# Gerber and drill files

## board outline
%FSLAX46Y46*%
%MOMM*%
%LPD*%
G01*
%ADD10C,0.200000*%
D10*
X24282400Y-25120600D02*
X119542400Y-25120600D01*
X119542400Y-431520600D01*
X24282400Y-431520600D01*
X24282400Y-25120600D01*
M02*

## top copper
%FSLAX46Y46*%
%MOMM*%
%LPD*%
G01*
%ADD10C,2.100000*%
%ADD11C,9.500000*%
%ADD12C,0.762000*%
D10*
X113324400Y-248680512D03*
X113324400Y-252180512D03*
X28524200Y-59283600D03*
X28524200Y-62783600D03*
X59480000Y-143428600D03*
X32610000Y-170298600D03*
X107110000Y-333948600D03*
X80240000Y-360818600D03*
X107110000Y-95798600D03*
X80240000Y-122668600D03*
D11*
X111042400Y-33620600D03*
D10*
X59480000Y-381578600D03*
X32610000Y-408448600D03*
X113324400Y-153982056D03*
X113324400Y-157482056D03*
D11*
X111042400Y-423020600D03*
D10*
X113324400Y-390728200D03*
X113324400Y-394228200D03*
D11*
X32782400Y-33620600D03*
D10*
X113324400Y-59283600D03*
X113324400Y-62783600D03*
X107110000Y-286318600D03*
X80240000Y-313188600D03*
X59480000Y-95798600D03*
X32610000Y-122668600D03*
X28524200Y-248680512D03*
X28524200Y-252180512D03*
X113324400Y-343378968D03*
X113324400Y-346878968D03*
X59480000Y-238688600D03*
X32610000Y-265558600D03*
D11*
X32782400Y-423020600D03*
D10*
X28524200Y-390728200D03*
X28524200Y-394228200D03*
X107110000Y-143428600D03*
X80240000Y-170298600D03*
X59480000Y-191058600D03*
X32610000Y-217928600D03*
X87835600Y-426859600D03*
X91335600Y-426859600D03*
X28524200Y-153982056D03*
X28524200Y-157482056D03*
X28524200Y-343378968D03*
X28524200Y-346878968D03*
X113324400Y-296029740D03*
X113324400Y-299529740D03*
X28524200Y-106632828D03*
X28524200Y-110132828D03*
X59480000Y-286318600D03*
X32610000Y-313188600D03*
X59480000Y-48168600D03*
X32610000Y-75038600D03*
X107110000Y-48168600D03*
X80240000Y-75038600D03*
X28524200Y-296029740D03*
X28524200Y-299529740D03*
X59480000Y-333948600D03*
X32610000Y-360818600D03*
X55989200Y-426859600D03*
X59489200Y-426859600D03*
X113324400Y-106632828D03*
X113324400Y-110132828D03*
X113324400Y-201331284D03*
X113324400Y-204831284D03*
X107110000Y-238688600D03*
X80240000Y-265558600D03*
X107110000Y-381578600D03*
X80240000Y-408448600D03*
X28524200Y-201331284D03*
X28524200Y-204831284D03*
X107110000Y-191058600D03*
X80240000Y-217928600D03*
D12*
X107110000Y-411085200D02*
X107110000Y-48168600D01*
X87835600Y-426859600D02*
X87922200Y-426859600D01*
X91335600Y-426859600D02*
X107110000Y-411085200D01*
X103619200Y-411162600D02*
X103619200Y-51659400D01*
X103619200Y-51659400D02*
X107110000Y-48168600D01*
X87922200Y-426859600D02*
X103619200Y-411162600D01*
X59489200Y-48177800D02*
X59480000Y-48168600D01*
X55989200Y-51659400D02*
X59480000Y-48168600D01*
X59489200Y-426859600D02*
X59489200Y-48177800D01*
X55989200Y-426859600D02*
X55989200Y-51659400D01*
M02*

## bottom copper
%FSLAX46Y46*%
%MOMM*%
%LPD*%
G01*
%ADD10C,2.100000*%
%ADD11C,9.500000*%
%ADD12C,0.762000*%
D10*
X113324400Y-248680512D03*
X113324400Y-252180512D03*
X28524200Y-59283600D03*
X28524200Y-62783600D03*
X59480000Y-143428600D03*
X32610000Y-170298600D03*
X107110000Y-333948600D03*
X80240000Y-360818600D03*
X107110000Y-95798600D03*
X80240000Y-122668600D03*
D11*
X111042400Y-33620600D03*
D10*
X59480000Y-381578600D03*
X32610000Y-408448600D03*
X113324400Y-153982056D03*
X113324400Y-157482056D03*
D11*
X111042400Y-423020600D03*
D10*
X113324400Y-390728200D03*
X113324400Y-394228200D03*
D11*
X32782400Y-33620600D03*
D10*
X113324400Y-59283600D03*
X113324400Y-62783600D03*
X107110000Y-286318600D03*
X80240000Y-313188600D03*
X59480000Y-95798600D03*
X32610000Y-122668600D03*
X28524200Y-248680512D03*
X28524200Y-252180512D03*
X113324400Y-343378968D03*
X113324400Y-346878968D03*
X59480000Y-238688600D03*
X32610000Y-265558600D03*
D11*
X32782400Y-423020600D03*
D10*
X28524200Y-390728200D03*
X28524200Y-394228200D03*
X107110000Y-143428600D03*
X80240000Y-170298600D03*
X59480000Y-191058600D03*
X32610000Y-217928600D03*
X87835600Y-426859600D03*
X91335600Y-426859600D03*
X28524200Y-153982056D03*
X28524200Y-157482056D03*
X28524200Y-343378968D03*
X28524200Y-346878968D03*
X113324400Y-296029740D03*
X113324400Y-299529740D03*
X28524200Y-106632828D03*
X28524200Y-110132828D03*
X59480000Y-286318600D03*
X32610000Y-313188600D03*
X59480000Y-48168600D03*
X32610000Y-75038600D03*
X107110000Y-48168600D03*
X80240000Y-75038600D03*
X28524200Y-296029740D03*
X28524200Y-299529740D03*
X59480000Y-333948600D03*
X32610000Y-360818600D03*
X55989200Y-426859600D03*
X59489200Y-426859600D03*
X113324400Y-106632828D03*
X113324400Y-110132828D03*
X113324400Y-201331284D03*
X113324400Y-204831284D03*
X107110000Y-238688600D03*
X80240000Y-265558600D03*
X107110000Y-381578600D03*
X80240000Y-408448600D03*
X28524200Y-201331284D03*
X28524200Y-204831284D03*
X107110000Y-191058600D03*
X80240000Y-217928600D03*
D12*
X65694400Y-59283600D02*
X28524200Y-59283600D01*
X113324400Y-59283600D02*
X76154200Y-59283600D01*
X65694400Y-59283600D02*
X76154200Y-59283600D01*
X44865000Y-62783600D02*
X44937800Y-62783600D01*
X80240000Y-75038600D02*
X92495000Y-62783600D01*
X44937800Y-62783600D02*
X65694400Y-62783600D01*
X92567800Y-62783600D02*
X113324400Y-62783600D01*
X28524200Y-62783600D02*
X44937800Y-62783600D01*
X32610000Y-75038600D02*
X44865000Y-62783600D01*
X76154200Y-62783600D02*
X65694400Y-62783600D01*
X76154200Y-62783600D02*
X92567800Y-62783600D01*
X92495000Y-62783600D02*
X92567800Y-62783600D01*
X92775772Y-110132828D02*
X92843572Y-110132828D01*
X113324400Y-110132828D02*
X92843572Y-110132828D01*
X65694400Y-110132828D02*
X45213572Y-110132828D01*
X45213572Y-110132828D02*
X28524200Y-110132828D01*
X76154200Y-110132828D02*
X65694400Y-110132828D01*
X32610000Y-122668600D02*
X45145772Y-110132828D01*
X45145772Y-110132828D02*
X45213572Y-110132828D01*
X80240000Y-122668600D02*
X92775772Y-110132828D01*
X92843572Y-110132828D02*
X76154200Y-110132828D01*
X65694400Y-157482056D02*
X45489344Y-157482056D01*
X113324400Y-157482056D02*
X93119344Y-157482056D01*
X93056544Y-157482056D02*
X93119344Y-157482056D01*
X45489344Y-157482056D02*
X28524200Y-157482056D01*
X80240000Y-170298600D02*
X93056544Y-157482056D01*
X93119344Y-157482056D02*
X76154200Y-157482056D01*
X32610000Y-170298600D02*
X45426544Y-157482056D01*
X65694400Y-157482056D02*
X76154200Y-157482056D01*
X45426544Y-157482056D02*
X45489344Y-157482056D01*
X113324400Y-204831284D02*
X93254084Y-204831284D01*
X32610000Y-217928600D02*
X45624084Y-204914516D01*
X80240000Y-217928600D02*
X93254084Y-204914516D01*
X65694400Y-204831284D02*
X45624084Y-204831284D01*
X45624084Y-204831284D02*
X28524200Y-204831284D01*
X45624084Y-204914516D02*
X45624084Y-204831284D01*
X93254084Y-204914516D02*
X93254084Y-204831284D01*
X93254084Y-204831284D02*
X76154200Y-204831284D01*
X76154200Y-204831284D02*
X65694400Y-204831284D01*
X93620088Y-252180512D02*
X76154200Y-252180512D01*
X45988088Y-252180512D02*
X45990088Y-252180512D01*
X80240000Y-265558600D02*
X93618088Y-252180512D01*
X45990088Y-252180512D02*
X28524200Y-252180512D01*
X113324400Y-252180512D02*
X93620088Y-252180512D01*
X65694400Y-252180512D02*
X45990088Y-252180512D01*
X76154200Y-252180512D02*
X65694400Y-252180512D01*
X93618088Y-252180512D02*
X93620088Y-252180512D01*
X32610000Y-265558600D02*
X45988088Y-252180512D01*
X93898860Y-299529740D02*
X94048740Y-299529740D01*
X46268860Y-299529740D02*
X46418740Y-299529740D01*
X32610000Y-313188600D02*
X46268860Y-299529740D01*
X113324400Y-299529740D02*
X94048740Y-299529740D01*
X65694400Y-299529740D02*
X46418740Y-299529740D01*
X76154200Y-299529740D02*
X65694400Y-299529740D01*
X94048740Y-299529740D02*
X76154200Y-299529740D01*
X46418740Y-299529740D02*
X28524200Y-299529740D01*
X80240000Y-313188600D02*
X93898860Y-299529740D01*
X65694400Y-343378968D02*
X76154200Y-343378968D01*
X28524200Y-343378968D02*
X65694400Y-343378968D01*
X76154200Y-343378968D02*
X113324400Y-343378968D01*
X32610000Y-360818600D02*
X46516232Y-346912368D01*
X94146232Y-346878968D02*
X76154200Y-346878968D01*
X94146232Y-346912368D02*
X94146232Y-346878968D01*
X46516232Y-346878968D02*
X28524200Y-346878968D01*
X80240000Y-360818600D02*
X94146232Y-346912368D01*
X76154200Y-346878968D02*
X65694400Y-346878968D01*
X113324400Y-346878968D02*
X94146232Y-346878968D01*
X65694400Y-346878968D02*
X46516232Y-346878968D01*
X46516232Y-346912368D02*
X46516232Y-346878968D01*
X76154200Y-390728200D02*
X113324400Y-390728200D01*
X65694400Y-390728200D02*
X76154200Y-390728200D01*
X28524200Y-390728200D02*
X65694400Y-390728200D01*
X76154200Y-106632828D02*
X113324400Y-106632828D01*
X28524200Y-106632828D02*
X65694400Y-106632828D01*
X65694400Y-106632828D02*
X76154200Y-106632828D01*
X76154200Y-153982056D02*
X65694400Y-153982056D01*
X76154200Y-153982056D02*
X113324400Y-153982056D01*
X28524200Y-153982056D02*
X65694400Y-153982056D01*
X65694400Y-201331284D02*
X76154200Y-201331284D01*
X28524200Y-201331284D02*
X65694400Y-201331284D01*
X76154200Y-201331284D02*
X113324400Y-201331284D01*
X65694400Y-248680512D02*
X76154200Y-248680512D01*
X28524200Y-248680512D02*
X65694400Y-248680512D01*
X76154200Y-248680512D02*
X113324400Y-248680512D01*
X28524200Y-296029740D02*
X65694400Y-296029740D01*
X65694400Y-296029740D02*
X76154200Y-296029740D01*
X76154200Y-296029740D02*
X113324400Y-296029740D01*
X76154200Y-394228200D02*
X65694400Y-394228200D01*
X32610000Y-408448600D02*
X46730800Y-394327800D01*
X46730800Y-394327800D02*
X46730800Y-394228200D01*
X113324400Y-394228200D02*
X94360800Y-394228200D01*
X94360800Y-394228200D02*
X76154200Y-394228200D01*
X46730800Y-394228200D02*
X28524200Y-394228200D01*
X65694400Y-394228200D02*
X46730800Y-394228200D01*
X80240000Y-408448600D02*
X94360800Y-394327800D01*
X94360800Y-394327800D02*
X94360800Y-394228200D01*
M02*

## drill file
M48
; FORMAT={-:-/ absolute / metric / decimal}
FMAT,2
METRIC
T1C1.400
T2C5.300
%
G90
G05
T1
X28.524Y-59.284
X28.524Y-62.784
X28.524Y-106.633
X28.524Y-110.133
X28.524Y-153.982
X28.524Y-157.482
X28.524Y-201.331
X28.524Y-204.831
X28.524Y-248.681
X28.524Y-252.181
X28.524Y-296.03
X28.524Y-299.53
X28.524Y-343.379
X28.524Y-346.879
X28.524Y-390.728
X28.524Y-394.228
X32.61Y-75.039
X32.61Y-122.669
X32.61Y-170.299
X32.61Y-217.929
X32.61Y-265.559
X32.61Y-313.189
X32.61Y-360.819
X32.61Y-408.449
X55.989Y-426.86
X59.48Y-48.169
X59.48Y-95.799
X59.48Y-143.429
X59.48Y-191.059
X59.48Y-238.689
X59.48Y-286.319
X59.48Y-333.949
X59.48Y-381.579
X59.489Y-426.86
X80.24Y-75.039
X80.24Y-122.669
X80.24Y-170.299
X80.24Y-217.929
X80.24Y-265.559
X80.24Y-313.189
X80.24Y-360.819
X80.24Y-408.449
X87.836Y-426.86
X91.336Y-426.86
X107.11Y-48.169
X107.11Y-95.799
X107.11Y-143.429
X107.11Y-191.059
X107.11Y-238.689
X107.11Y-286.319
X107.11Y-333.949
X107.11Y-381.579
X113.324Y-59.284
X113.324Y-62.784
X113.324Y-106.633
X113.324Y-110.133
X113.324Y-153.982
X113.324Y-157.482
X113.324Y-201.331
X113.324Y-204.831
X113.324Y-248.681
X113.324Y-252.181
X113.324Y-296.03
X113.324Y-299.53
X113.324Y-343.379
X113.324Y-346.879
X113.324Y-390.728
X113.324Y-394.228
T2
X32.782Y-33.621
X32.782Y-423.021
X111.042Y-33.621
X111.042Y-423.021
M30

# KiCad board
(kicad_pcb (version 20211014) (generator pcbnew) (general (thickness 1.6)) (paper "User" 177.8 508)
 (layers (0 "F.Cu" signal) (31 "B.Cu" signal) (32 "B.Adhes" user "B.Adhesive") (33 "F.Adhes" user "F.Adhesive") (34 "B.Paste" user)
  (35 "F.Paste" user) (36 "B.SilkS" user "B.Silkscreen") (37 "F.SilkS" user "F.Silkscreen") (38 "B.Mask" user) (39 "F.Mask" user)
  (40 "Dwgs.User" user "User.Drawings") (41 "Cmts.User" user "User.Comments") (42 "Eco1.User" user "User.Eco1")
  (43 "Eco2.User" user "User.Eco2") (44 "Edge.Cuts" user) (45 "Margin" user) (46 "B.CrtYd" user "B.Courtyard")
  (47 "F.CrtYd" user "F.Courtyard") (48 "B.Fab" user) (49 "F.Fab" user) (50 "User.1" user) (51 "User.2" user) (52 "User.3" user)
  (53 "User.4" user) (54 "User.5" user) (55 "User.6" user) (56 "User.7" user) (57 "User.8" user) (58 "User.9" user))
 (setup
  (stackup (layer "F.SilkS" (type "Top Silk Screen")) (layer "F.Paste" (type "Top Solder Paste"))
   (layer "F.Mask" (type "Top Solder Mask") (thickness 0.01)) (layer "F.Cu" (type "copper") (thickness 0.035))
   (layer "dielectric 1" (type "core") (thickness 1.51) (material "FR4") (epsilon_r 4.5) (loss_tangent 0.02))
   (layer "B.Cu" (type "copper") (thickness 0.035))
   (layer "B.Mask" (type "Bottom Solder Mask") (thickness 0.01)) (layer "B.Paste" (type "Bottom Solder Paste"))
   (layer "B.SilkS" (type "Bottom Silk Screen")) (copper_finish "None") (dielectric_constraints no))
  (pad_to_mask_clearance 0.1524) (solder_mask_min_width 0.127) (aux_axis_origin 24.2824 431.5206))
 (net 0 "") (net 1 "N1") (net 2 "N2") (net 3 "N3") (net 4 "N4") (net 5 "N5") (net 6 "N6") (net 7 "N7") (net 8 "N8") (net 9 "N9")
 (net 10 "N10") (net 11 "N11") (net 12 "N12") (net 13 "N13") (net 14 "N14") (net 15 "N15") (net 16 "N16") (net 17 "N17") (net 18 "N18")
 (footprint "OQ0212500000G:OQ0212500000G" (layer "F.Cu") (at 113.3244 248.680512 -90)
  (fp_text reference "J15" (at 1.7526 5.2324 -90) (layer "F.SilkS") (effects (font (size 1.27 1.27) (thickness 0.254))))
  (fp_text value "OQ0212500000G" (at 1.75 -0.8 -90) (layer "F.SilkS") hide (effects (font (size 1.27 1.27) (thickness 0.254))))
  (pad "1" thru_hole circle (at 0 0 270) (size 2.1 2.1) (drill 1.4) (layers F&B.Cu *.Mask) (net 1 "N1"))
  (pad "2" thru_hole circle (at 3.5 0 270) (size 2.1 2.1) (drill 1.4) (layers F&B.Cu *.Mask) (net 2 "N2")))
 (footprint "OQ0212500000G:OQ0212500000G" (layer "F.Cu") (at 28.5242 59.2836 -90)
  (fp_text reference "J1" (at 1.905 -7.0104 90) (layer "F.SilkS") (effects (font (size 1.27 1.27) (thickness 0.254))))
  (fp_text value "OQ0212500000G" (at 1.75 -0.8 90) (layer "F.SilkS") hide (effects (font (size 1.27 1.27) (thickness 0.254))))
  (pad "1" thru_hole circle (at 0 0 270) (size 2.1 2.1) (drill 1.4) (layers *.Cu *.Mask) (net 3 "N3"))
  (pad "2" thru_hole circle (at 3.5 0 270) (size 2.1 2.1) (drill 1.4) (layers *.Cu *.Mask) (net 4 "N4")))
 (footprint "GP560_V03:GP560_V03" (layer "F.Cu") (at 32.61 170.2986)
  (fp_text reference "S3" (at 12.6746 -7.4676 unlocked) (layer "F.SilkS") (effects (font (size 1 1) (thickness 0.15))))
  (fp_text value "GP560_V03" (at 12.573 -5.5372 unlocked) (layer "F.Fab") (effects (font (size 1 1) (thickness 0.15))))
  (pad "1" thru_hole circle (at 26.87 -26.87) (size 2.1 2.1) (drill 1.4) (layers *.Cu *.Mask) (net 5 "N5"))
  (pad "2" thru_hole circle (at 0 0) (size 2.1 2.1) (drill 1.4) (layers *.Cu *.Mask) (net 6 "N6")))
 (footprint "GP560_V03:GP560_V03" (layer "F.Cu") (at 80.24 360.8186)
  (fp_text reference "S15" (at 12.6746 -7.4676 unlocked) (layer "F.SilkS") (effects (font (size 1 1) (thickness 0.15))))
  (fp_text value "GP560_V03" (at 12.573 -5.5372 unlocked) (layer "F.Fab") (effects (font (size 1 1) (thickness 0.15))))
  (pad "1" thru_hole circle (at 26.87 -26.87) (size 2.1 2.1) (drill 1.4) (layers *.Cu *.Mask) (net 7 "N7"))
  (pad "2" thru_hole circle (at 0 0) (size 2.1 2.1) (drill 1.4) (layers *.Cu *.Mask) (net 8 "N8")))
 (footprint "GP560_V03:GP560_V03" (layer "F.Cu") (at 80.24 122.6686)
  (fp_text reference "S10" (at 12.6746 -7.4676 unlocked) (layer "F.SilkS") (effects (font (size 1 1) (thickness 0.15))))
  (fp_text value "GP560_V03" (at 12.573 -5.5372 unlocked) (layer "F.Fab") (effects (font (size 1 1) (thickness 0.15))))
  (pad "1" thru_hole circle (at 26.87 -26.87) (size 2.1 2.1) (drill 1.4) (layers *.Cu *.Mask) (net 7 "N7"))
  (pad "2" thru_hole circle (at 0 0) (size 2.1 2.1) (drill 1.4) (layers *.Cu *.Mask) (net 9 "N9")))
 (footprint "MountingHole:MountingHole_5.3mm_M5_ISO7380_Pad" (layer "F.Cu") (at 111.0424 33.6206)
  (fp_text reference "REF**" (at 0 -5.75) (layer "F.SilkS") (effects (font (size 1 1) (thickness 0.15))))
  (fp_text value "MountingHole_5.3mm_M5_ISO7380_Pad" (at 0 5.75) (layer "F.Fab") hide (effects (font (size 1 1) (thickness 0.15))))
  (pad "1" thru_hole circle (at 0 0) (size 9.5 9.5) (drill 5.3) (layers F&B.Cu *.Mask)))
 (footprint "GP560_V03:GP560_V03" (layer "F.Cu") (at 32.61 408.4486)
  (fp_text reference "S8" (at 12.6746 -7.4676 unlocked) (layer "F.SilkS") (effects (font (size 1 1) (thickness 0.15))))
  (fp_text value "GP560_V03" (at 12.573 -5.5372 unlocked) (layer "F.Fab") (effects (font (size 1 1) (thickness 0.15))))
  (pad "1" thru_hole circle (at 26.87 -26.87) (size 2.1 2.1) (drill 1.4) (layers *.Cu *.Mask) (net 5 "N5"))
  (pad "2" thru_hole circle (at 0 0) (size 2.1 2.1) (drill 1.4) (layers *.Cu *.Mask) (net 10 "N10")))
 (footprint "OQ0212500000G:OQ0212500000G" (layer "F.Cu") (at 113.3244 153.982056 -90)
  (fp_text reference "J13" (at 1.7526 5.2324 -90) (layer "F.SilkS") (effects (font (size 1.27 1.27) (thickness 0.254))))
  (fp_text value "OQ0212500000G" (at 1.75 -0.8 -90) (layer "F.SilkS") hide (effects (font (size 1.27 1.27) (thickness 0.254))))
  (pad "1" thru_hole circle (at 0 0 270) (size 2.1 2.1) (drill 1.4) (layers F&B.Cu *.Mask) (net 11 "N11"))
  (pad "2" thru_hole circle (at 3.5 0 270) (size 2.1 2.1) (drill 1.4) (layers F&B.Cu *.Mask) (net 6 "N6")))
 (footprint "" (layer "F.Cu") (at 111.0424 423.0206)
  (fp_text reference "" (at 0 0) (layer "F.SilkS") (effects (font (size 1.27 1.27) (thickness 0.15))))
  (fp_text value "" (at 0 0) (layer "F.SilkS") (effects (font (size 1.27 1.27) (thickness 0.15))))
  (pad "1" thru_hole circle (at 0 0) (size 9.5 9.5) (drill 5.3) (layers F&B.Cu *.Mask)))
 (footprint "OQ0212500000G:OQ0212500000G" (layer "F.Cu") (at 113.3244 390.7282 -90)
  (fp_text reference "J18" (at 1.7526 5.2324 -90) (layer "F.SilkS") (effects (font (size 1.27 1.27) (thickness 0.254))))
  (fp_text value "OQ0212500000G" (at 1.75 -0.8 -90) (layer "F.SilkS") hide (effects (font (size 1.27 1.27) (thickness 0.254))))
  (pad "1" thru_hole circle (at 0 0 270) (size 2.1 2.1) (drill 1.4) (layers F&B.Cu *.Mask) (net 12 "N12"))
  (pad "2" thru_hole circle (at 3.5 0 270) (size 2.1 2.1) (drill 1.4) (layers F&B.Cu *.Mask) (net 10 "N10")))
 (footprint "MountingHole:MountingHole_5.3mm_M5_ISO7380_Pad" (layer "F.Cu") (at 32.7824 33.6206)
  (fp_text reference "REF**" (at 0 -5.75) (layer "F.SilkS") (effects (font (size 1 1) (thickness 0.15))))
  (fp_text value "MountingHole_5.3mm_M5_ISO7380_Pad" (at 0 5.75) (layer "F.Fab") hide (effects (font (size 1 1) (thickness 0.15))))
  (pad "1" thru_hole circle (at 0 0) (size 9.5 9.5) (drill 5.3) (layers F&B.Cu *.Mask)))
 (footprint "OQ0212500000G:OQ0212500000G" (layer "F.Cu") (at 113.3244 59.2836 -90)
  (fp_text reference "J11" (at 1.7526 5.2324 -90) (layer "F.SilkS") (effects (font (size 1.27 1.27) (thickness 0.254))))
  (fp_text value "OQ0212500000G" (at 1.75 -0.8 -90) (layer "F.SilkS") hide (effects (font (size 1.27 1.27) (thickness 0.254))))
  (pad "1" thru_hole circle (at 0 0 270) (size 2.1 2.1) (drill 1.4) (layers F&B.Cu *.Mask) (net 3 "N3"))
  (pad "2" thru_hole circle (at 3.5 0 270) (size 2.1 2.1) (drill 1.4) (layers F&B.Cu *.Mask) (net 4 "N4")))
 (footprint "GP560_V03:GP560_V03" (layer "F.Cu") (at 80.24 313.1886)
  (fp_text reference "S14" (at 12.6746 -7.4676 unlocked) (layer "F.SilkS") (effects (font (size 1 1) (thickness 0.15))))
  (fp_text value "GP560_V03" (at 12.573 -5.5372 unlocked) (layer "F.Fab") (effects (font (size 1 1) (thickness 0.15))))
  (pad "1" thru_hole circle (at 26.87 -26.87) (size 2.1 2.1) (drill 1.4) (layers *.Cu *.Mask) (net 7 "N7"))
  (pad "2" thru_hole circle (at 0 0) (size 2.1 2.1) (drill 1.4) (layers *.Cu *.Mask) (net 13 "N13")))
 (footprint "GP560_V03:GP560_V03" (layer "F.Cu") (at 32.61 122.6686)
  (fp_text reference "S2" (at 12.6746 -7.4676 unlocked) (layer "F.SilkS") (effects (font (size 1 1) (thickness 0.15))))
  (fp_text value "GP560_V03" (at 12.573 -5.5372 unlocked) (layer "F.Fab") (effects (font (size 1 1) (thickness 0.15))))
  (pad "1" thru_hole circle (at 26.87 -26.87) (size 2.1 2.1) (drill 1.4) (layers *.Cu *.Mask) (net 5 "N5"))
  (pad "2" thru_hole circle (at 0 0) (size 2.1 2.1) (drill 1.4) (layers *.Cu *.Mask) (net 9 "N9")))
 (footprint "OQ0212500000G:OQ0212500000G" (layer "F.Cu") (at 28.5242 248.680512 -90)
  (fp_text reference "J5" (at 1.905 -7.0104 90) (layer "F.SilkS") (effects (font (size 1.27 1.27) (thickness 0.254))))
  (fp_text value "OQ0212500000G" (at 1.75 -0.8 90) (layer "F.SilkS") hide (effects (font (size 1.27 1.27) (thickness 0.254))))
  (pad "1" thru_hole circle (at 0 0 270) (size 2.1 2.1) (drill 1.4) (layers *.Cu *.Mask) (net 1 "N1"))
  (pad "2" thru_hole circle (at 3.5 0 270) (size 2.1 2.1) (drill 1.4) (layers *.Cu *.Mask) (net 2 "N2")))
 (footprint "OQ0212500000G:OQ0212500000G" (layer "F.Cu") (at 113.3244 343.378968 -90)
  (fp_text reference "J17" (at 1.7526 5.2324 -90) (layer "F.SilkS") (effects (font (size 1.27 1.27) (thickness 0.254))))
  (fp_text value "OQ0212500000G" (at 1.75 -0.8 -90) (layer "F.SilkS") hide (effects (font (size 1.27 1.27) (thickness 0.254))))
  (pad "1" thru_hole circle (at 0 0 270) (size 2.1 2.1) (drill 1.4) (layers F&B.Cu *.Mask) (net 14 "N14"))
  (pad "2" thru_hole circle (at 3.5 0 270) (size 2.1 2.1) (drill 1.4) (layers F&B.Cu *.Mask) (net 8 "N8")))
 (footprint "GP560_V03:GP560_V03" (layer "F.Cu") (at 32.61 265.5586)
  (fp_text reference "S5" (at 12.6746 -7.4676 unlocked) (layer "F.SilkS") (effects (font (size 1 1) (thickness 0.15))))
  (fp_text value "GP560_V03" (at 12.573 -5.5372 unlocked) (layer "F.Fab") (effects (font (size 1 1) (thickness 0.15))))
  (pad "1" thru_hole circle (at 26.87 -26.87) (size 2.1 2.1) (drill 1.4) (layers *.Cu *.Mask) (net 5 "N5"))
  (pad "2" thru_hole circle (at 0 0) (size 2.1 2.1) (drill 1.4) (layers *.Cu *.Mask) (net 2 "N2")))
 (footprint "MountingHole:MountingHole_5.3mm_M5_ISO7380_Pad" (layer "F.Cu") (at 32.7824 423.0206)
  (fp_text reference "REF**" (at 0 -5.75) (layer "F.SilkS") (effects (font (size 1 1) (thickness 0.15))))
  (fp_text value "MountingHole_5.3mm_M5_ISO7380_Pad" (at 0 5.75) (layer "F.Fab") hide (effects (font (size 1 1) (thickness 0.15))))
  (pad "1" thru_hole circle (at 0 0) (size 9.5 9.5) (drill 5.3) (layers *.Cu *.Mask)))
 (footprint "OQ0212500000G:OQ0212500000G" (layer "F.Cu") (at 28.5242 390.7282 -90)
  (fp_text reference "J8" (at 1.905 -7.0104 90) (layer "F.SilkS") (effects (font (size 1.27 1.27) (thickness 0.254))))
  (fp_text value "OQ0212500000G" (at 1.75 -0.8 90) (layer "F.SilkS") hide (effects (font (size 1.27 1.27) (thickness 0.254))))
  (pad "1" thru_hole circle (at 0 0 270) (size 2.1 2.1) (drill 1.4) (layers *.Cu *.Mask) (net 12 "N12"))
  (pad "2" thru_hole circle (at 3.5 0 270) (size 2.1 2.1) (drill 1.4) (layers *.Cu *.Mask) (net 10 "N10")))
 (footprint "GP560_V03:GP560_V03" (layer "F.Cu") (at 80.24 170.2986)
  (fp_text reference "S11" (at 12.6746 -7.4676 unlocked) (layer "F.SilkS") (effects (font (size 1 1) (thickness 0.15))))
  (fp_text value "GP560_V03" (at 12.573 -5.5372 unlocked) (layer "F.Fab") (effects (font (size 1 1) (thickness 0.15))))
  (pad "1" thru_hole circle (at 26.87 -26.87) (size 2.1 2.1) (drill 1.4) (layers *.Cu *.Mask) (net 7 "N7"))
  (pad "2" thru_hole circle (at 0 0) (size 2.1 2.1) (drill 1.4) (layers *.Cu *.Mask) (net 6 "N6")))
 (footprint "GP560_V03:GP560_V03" (layer "F.Cu") (at 32.61 217.9286)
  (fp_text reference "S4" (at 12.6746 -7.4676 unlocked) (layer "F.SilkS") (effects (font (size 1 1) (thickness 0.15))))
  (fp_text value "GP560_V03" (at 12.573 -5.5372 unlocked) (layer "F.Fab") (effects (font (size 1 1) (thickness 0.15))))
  (pad "1" thru_hole circle (at 26.87 -26.87) (size 2.1 2.1) (drill 1.4) (layers *.Cu *.Mask) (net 5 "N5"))
  (pad "2" thru_hole circle (at 0 0) (size 2.1 2.1) (drill 1.4) (layers *.Cu *.Mask) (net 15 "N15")))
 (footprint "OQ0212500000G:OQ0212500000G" (layer "F.Cu") (at 87.8356 426.8596)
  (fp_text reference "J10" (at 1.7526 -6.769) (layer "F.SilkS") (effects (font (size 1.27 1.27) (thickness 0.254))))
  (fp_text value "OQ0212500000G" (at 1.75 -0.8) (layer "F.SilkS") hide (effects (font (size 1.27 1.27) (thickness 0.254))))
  (pad "1" thru_hole circle (at 0 0) (size 2.1 2.1) (drill 1.4) (layers *.Cu *.Mask) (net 7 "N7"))
  (pad "2" thru_hole circle (at 3.5 0) (size 2.1 2.1) (drill 1.4) (layers *.Cu *.Mask) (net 7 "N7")))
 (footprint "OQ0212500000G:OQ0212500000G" (layer "F.Cu") (at 28.5242 153.982056 -90)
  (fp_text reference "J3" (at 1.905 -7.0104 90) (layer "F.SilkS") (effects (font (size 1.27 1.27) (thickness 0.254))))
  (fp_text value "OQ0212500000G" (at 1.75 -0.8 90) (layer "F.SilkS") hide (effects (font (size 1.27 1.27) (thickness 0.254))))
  (pad "1" thru_hole circle (at 0 0 270) (size 2.1 2.1) (drill 1.4) (layers *.Cu *.Mask) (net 11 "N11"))
  (pad "2" thru_hole circle (at 3.5 0 270) (size 2.1 2.1) (drill 1.4) (layers *.Cu *.Mask) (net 6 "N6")))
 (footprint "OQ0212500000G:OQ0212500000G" (layer "F.Cu") (at 28.5242 343.378968 -90)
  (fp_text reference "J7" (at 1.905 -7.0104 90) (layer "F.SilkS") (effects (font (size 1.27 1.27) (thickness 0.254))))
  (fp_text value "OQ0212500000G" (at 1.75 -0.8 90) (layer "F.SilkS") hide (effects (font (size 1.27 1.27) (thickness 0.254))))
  (pad "1" thru_hole circle (at 0 0 270) (size 2.1 2.1) (drill 1.4) (layers *.Cu *.Mask) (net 14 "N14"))
  (pad "2" thru_hole circle (at 3.5 0 270) (size 2.1 2.1) (drill 1.4) (layers *.Cu *.Mask) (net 8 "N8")))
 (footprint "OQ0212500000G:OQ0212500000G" (layer "F.Cu") (at 113.3244 296.02974 -90)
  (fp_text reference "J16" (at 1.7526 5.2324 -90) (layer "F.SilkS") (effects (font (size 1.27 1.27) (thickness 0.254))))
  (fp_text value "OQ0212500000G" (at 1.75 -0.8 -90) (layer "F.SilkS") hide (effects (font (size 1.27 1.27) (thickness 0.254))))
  (pad "1" thru_hole circle (at 0 0 270) (size 2.1 2.1) (drill 1.4) (layers F&B.Cu *.Mask) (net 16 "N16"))
  (pad "2" thru_hole circle (at 3.5 0 270) (size 2.1 2.1) (drill 1.4) (layers F&B.Cu *.Mask) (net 13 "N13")))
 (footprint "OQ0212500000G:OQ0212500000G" (layer "F.Cu") (at 28.5242 106.632828 -90)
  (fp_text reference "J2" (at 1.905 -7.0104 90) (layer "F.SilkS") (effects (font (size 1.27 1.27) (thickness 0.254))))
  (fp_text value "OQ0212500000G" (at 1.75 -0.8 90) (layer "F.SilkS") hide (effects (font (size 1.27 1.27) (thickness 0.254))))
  (pad "1" thru_hole circle (at 0 0 270) (size 2.1 2.1) (drill 1.4) (layers *.Cu *.Mask) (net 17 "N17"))
  (pad "2" thru_hole circle (at 3.5 0 270) (size 2.1 2.1) (drill 1.4) (layers *.Cu *.Mask) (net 9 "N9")))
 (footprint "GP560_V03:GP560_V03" (layer "F.Cu") (at 32.61 313.1886)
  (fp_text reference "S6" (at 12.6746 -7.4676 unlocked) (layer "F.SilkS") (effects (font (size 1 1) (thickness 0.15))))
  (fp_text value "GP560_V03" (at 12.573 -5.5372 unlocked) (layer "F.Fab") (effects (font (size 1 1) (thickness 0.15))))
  (pad "1" thru_hole circle (at 26.87 -26.87) (size 2.1 2.1) (drill 1.4) (layers *.Cu *.Mask) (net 5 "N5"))
  (pad "2" thru_hole circle (at 0 0) (size 2.1 2.1) (drill 1.4) (layers *.Cu *.Mask) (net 13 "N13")))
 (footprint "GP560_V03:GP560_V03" (layer "F.Cu") (at 32.61 75.0386)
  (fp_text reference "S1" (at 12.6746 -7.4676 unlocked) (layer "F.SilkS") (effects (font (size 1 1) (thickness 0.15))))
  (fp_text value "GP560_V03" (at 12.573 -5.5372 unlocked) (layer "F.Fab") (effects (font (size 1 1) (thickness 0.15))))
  (pad "1" thru_hole circle (at 26.87 -26.87) (size 2.1 2.1) (drill 1.4) (layers *.Cu *.Mask) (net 5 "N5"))
  (pad "2" thru_hole circle (at 0 0) (size 2.1 2.1) (drill 1.4) (layers *.Cu *.Mask) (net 4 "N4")))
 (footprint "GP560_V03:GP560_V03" (layer "F.Cu") (at 80.24 75.0386)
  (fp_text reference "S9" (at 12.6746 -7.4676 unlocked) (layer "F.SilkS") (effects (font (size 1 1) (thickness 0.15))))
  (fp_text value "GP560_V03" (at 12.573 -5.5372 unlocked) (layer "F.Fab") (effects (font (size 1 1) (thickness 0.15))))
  (pad "1" thru_hole circle (at 26.87 -26.87) (size 2.1 2.1) (drill 1.4) (layers *.Cu *.Mask) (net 7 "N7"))
  (pad "2" thru_hole circle (at 0 0) (size 2.1 2.1) (drill 1.4) (layers *.Cu *.Mask) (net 4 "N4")))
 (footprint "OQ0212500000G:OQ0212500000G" (layer "F.Cu") (at 28.5242 296.02974 -90)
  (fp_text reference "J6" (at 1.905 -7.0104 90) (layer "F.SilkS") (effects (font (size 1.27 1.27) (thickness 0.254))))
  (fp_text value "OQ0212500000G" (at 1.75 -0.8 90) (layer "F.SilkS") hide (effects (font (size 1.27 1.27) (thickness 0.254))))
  (pad "1" thru_hole circle (at 0 0 270) (size 2.1 2.1) (drill 1.4) (layers *.Cu *.Mask) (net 16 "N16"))
  (pad "2" thru_hole circle (at 3.5 0 270) (size 2.1 2.1) (drill 1.4) (layers *.Cu *.Mask) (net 13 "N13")))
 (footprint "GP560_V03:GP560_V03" (layer "F.Cu") (at 32.61 360.8186)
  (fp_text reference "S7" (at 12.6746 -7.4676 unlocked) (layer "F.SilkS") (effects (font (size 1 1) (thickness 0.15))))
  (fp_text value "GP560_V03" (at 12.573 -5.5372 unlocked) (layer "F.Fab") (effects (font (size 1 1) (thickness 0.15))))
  (pad "1" thru_hole circle (at 26.87 -26.87) (size 2.1 2.1) (drill 1.4) (layers *.Cu *.Mask) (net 5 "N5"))
  (pad "2" thru_hole circle (at 0 0) (size 2.1 2.1) (drill 1.4) (layers *.Cu *.Mask) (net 8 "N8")))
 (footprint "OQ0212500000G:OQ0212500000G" (layer "F.Cu") (at 55.9892 426.8596)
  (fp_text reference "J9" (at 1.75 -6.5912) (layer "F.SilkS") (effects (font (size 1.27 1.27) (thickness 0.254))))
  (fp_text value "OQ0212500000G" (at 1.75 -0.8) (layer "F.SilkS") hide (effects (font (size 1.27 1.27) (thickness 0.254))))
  (pad "1" thru_hole circle (at 0 0) (size 2.1 2.1) (drill 1.4) (layers *.Cu *.Mask) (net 5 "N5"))
  (pad "2" thru_hole circle (at 3.5 0) (size 2.1 2.1) (drill 1.4) (layers *.Cu *.Mask) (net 5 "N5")))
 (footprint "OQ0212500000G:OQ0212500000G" (layer "F.Cu") (at 113.3244 106.632828 -90)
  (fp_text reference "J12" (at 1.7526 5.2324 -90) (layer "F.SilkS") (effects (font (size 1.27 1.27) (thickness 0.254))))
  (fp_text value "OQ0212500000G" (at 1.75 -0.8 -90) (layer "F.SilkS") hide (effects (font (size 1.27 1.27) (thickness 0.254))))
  (pad "1" thru_hole circle (at 0 0 270) (size 2.1 2.1) (drill 1.4) (layers F&B.Cu *.Mask) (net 17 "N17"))
  (pad "2" thru_hole circle (at 3.5 0 270) (size 2.1 2.1) (drill 1.4) (layers F&B.Cu *.Mask) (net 9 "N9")))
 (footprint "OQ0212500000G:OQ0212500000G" (layer "F.Cu") (at 113.3244 201.331284 -90)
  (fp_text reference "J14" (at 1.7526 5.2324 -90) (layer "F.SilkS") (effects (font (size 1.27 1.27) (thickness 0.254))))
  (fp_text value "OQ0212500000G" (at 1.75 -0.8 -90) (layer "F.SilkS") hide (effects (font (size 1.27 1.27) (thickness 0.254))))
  (pad "1" thru_hole circle (at 0 0 270) (size 2.1 2.1) (drill 1.4) (layers F&B.Cu *.Mask) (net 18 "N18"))
  (pad "2" thru_hole circle (at 3.5 0 270) (size 2.1 2.1) (drill 1.4) (layers F&B.Cu *.Mask) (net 15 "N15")))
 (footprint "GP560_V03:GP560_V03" (layer "F.Cu") (at 80.24 265.5586)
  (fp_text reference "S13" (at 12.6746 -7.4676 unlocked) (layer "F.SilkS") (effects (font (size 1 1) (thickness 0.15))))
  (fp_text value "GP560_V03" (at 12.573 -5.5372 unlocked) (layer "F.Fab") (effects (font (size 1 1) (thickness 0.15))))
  (pad "1" thru_hole circle (at 26.87 -26.87) (size 2.1 2.1) (drill 1.4) (layers *.Cu *.Mask) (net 7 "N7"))
  (pad "2" thru_hole circle (at 0 0) (size 2.1 2.1) (drill 1.4) (layers *.Cu *.Mask) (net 2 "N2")))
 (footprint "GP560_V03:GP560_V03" (layer "F.Cu") (at 80.24 408.4486)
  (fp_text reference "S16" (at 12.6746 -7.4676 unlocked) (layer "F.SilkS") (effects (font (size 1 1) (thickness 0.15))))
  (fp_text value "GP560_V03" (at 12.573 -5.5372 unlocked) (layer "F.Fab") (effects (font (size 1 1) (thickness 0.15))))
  (pad "1" thru_hole circle (at 26.87 -26.87) (size 2.1 2.1) (drill 1.4) (layers *.Cu *.Mask) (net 7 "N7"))
  (pad "2" thru_hole circle (at 0 0) (size 2.1 2.1) (drill 1.4) (layers *.Cu *.Mask) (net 10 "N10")))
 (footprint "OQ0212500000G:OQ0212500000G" (layer "F.Cu") (at 28.5242 201.331284 -90)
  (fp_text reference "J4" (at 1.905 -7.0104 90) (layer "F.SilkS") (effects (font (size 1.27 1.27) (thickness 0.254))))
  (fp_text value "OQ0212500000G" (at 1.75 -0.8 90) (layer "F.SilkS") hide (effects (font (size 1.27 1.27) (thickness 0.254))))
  (pad "1" thru_hole circle (at 0 0 270) (size 2.1 2.1) (drill 1.4) (layers *.Cu *.Mask) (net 18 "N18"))
  (pad "2" thru_hole circle (at 3.5 0 270) (size 2.1 2.1) (drill 1.4) (layers *.Cu *.Mask) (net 15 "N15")))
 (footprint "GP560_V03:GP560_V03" (layer "F.Cu") (at 80.24 217.9286)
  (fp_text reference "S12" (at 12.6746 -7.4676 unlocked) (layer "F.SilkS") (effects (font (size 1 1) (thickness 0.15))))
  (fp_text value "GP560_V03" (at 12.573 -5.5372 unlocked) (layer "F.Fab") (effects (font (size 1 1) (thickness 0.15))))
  (pad "1" thru_hole circle (at 26.87 -26.87) (size 2.1 2.1) (drill 1.4) (layers *.Cu *.Mask) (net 7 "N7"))
  (pad "2" thru_hole circle (at 0 0) (size 2.1 2.1) (drill 1.4) (layers *.Cu *.Mask) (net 15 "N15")))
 (gr_rect (start 24.2824 431.5206) (end 119.5424 25.1206) (layer "Edge.Cuts") (width 0.2) (fill none))
 (segment (start 65.6944 59.2836) (end 28.5242 59.2836) (width 0.762) (layer "B.Cu") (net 3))
 (segment (start 113.3244 59.2836) (end 76.1542 59.2836) (width 0.762) (layer "B.Cu") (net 3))
 (segment (start 65.6944 59.2836) (end 76.1542 59.2836) (width 0.762) (layer "B.Cu") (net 3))
 (segment (start 44.865 62.7836) (end 44.9378 62.7836) (width 0.762) (layer "B.Cu") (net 4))
 (segment (start 80.24 75.0386) (end 92.495 62.7836) (width 0.762) (layer "B.Cu") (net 4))
 (segment (start 44.9378 62.7836) (end 65.6944 62.7836) (width 0.762) (layer "B.Cu") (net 4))
 (segment (start 92.5678 62.7836) (end 113.3244 62.7836) (width 0.762) (layer "B.Cu") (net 4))
 (segment (start 28.5242 62.7836) (end 44.9378 62.7836) (width 0.762) (layer "B.Cu") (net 4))
 (segment (start 32.61 75.0386) (end 44.865 62.7836) (width 0.762) (layer "B.Cu") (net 4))
 (segment (start 76.1542 62.7836) (end 65.6944 62.7836) (width 0.762) (layer "B.Cu") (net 4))
 (segment (start 76.1542 62.7836) (end 92.5678 62.7836) (width 0.762) (layer "B.Cu") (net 4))
 (segment (start 92.495 62.7836) (end 92.5678 62.7836) (width 0.762) (layer "B.Cu") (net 4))
 (segment (start 92.775772 110.132828) (end 92.843572 110.132828) (width 0.762) (layer "B.Cu") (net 9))
 (segment (start 113.3244 110.132828) (end 92.843572 110.132828) (width 0.762) (layer "B.Cu") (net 9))
 (segment (start 65.6944 110.132828) (end 45.213572 110.132828) (width 0.762) (layer "B.Cu") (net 9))
 (segment (start 45.213572 110.132828) (end 28.5242 110.132828) (width 0.762) (layer "B.Cu") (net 9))
 (segment (start 76.1542 110.132828) (end 65.6944 110.132828) (width 0.762) (layer "B.Cu") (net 9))
 (segment (start 32.61 122.6686) (end 45.145772 110.132828) (width 0.762) (layer "B.Cu") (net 9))
 (segment (start 45.145772 110.132828) (end 45.213572 110.132828) (width 0.762) (layer "B.Cu") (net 9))
 (segment (start 80.24 122.6686) (end 92.775772 110.132828) (width 0.762) (layer "B.Cu") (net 9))
 (segment (start 92.843572 110.132828) (end 76.1542 110.132828) (width 0.762) (layer "B.Cu") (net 9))
 (segment (start 65.6944 157.482056) (end 45.489344 157.482056) (width 0.762) (layer "B.Cu") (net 6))
 (segment (start 113.3244 157.482056) (end 93.119344 157.482056) (width 0.762) (layer "B.Cu") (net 6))
 (segment (start 93.056544 157.482056) (end 93.119344 157.482056) (width 0.762) (layer "B.Cu") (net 6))
 (segment (start 45.489344 157.482056) (end 28.5242 157.482056) (width 0.762) (layer "B.Cu") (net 6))
 (segment (start 80.24 170.2986) (end 93.056544 157.482056) (width 0.762) (layer "B.Cu") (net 6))
 (segment (start 93.119344 157.482056) (end 76.1542 157.482056) (width 0.762) (layer "B.Cu") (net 6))
 (segment (start 32.61 170.2986) (end 45.426544 157.482056) (width 0.762) (layer "B.Cu") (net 6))
 (segment (start 65.6944 157.482056) (end 76.1542 157.482056) (width 0.762) (layer "B.Cu") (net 6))
 (segment (start 45.426544 157.482056) (end 45.489344 157.482056) (width 0.762) (layer "B.Cu") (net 6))
 (segment (start 113.3244 204.831284) (end 93.254084 204.831284) (width 0.762) (layer "B.Cu") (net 15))
 (segment (start 32.61 217.9286) (end 45.624084 204.914516) (width 0.762) (layer "B.Cu") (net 15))
 (segment (start 80.24 217.9286) (end 93.254084 204.914516) (width 0.762) (layer "B.Cu") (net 15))
 (segment (start 65.6944 204.831284) (end 45.624084 204.831284) (width 0.762) (layer "B.Cu") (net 15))
 (segment (start 45.624084 204.831284) (end 28.5242 204.831284) (width 0.762) (layer "B.Cu") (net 15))
 (segment (start 45.624084 204.914516) (end 45.624084 204.831284) (width 0.762) (layer "B.Cu") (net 15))
 (segment (start 93.254084 204.914516) (end 93.254084 204.831284) (width 0.762) (layer "B.Cu") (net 15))
 (segment (start 93.254084 204.831284) (end 76.1542 204.831284) (width 0.762) (layer "B.Cu") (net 15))
 (segment (start 76.1542 204.831284) (end 65.6944 204.831284) (width 0.762) (layer "B.Cu") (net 15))
 (segment (start 93.620088 252.180512) (end 76.1542 252.180512) (width 0.762) (layer "B.Cu") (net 2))
 (segment (start 45.988088 252.180512) (end 45.990088 252.180512) (width 0.762) (layer "B.Cu") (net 2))
 (segment (start 80.24 265.5586) (end 93.618088 252.180512) (width 0.762) (layer "B.Cu") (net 2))
 (segment (start 45.990088 252.180512) (end 28.5242 252.180512) (width 0.762) (layer "B.Cu") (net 2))
 (segment (start 113.3244 252.180512) (end 93.620088 252.180512) (width 0.762) (layer "B.Cu") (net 2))
 (segment (start 65.6944 252.180512) (end 45.990088 252.180512) (width 0.762) (layer "B.Cu") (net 2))
 (segment (start 76.1542 252.180512) (end 65.6944 252.180512) (width 0.762) (layer "B.Cu") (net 2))
 (segment (start 93.618088 252.180512) (end 93.620088 252.180512) (width 0.762) (layer "B.Cu") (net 2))
 (segment (start 32.61 265.5586) (end 45.988088 252.180512) (width 0.762) (layer "B.Cu") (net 2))
 (segment (start 93.89886 299.52974) (end 94.04874 299.52974) (width 0.762) (layer "B.Cu") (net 13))
 (segment (start 46.26886 299.52974) (end 46.41874 299.52974) (width 0.762) (layer "B.Cu") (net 13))
 (segment (start 32.61 313.1886) (end 46.26886 299.52974) (width 0.762) (layer "B.Cu") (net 13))
 (segment (start 113.3244 299.52974) (end 94.04874 299.52974) (width 0.762) (layer "B.Cu") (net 13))
 (segment (start 65.6944 299.52974) (end 46.41874 299.52974) (width 0.762) (layer "B.Cu") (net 13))
 (segment (start 76.1542 299.52974) (end 65.6944 299.52974) (width 0.762) (layer "B.Cu") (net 13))
 (segment (start 94.04874 299.52974) (end 76.1542 299.52974) (width 0.762) (layer "B.Cu") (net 13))
 (segment (start 46.41874 299.52974) (end 28.5242 299.52974) (width 0.762) (layer "B.Cu") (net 13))
 (segment (start 80.24 313.1886) (end 93.89886 299.52974) (width 0.762) (layer "B.Cu") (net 13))
 (segment (start 65.6944 343.378968) (end 76.1542 343.378968) (width 0.762) (layer "B.Cu") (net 14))
 (segment (start 28.5242 343.378968) (end 65.6944 343.378968) (width 0.762) (layer "B.Cu") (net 14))
 (segment (start 76.1542 343.378968) (end 113.3244 343.378968) (width 0.762) (layer "B.Cu") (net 14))
 (segment (start 32.61 360.8186) (end 46.516232 346.912368) (width 0.762) (layer "B.Cu") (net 8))
 (segment (start 94.146232 346.878968) (end 76.1542 346.878968) (width 0.762) (layer "B.Cu") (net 8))
 (segment (start 94.146232 346.912368) (end 94.146232 346.878968) (width 0.762) (layer "B.Cu") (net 8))
 (segment (start 46.516232 346.878968) (end 28.5242 346.878968) (width 0.762) (layer "B.Cu") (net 8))
 (segment (start 80.24 360.8186) (end 94.146232 346.912368) (width 0.762) (layer "B.Cu") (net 8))
 (segment (start 76.1542 346.878968) (end 65.6944 346.878968) (width 0.762) (layer "B.Cu") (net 8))
 (segment (start 113.3244 346.878968) (end 94.146232 346.878968) (width 0.762) (layer "B.Cu") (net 8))
 (segment (start 65.6944 346.878968) (end 46.516232 346.878968) (width 0.762) (layer "B.Cu") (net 8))
 (segment (start 46.516232 346.912368) (end 46.516232 346.878968) (width 0.762) (layer "B.Cu") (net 8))
 (segment (start 107.11 411.0852) (end 107.11 48.1686) (width 0.762) (layer "F.Cu") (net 7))
 (segment (start 87.8356 426.8596) (end 87.9222 426.8596) (width 0.762) (layer "F.Cu") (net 7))
 (segment (start 91.3356 426.8596) (end 107.11 411.0852) (width 0.762) (layer "F.Cu") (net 7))
 (segment (start 103.6192 411.1626) (end 103.6192 51.6594) (width 0.762) (layer "F.Cu") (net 7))
 (segment (start 103.6192 51.6594) (end 107.11 48.1686) (width 0.762) (layer "F.Cu") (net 7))
 (segment (start 87.9222 426.8596) (end 103.6192 411.1626) (width 0.762) (layer "F.Cu") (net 7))
 (segment (start 76.1542 390.7282) (end 113.3244 390.7282) (width 0.762) (layer "B.Cu") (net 12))
 (segment (start 65.6944 390.7282) (end 76.1542 390.7282) (width 0.762) (layer "B.Cu") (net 12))
 (segment (start 28.5242 390.7282) (end 65.6944 390.7282) (width 0.762) (layer "B.Cu") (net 12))
 (segment (start 76.1542 106.632828) (end 113.3244 106.632828) (width 0.762) (layer "B.Cu") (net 17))
 (segment (start 28.5242 106.632828) (end 65.6944 106.632828) (width 0.762) (layer "B.Cu") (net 17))
 (segment (start 65.6944 106.632828) (end 76.1542 106.632828) (width 0.762) (layer "B.Cu") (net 17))
 (segment (start 76.1542 153.982056) (end 65.6944 153.982056) (width 0.762) (layer "B.Cu") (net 11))
 (segment (start 76.1542 153.982056) (end 113.3244 153.982056) (width 0.762) (layer "B.Cu") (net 11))
 (segment (start 28.5242 153.982056) (end 65.6944 153.982056) (width 0.762) (layer "B.Cu") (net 11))
 (segment (start 65.6944 201.331284) (end 76.1542 201.331284) (width 0.762) (layer "B.Cu") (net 18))
 (segment (start 28.5242 201.331284) (end 65.6944 201.331284) (width 0.762) (layer "B.Cu") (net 18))
 (segment (start 76.1542 201.331284) (end 113.3244 201.331284) (width 0.762) (layer "B.Cu") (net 18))
 (segment (start 65.6944 248.680512) (end 76.1542 248.680512) (width 0.762) (layer "B.Cu") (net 1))
 (segment (start 28.5242 248.680512) (end 65.6944 248.680512) (width 0.762) (layer "B.Cu") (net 1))
 (segment (start 76.1542 248.680512) (end 113.3244 248.680512) (width 0.762) (layer "B.Cu") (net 1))
 (segment (start 28.5242 296.02974) (end 65.6944 296.02974) (width 0.762) (layer "B.Cu") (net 16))
 (segment (start 65.6944 296.02974) (end 76.1542 296.02974) (width 0.762) (layer "B.Cu") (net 16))
 (segment (start 76.1542 296.02974) (end 113.3244 296.02974) (width 0.762) (layer "B.Cu") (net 16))
 (segment (start 76.1542 394.2282) (end 65.6944 394.2282) (width 0.762) (layer "B.Cu") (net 10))
 (segment (start 32.61 408.4486) (end 46.7308 394.3278) (width 0.762) (layer "B.Cu") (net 10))
 (segment (start 46.7308 394.3278) (end 46.7308 394.2282) (width 0.762) (layer "B.Cu") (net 10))
 (segment (start 113.3244 394.2282) (end 94.3608 394.2282) (width 0.762) (layer "B.Cu") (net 10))
 (segment (start 94.3608 394.2282) (end 76.1542 394.2282) (width 0.762) (layer "B.Cu") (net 10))
 (segment (start 46.7308 394.2282) (end 28.5242 394.2282) (width 0.762) (layer "B.Cu") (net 10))
 (segment (start 65.6944 394.2282) (end 46.7308 394.2282) (width 0.762) (layer "B.Cu") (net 10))
 (segment (start 80.24 408.4486) (end 94.3608 394.3278) (width 0.762) (layer "B.Cu") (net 10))
 (segment (start 94.3608 394.3278) (end 94.3608 394.2282) (width 0.762) (layer "B.Cu") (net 10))
 (segment (start 59.4892 48.1778) (end 59.48 48.1686) (width 0.762) (layer "F.Cu") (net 5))
 (segment (start 55.9892 51.6594) (end 59.48 48.1686) (width 0.762) (layer "F.Cu") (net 5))
 (segment (start 59.4892 426.8596) (end 59.4892 48.1778) (width 0.762) (layer "F.Cu") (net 5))
 (segment (start 55.9892 426.8596) (end 55.9892 51.6594) (width 0.762) (layer "F.Cu") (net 5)))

